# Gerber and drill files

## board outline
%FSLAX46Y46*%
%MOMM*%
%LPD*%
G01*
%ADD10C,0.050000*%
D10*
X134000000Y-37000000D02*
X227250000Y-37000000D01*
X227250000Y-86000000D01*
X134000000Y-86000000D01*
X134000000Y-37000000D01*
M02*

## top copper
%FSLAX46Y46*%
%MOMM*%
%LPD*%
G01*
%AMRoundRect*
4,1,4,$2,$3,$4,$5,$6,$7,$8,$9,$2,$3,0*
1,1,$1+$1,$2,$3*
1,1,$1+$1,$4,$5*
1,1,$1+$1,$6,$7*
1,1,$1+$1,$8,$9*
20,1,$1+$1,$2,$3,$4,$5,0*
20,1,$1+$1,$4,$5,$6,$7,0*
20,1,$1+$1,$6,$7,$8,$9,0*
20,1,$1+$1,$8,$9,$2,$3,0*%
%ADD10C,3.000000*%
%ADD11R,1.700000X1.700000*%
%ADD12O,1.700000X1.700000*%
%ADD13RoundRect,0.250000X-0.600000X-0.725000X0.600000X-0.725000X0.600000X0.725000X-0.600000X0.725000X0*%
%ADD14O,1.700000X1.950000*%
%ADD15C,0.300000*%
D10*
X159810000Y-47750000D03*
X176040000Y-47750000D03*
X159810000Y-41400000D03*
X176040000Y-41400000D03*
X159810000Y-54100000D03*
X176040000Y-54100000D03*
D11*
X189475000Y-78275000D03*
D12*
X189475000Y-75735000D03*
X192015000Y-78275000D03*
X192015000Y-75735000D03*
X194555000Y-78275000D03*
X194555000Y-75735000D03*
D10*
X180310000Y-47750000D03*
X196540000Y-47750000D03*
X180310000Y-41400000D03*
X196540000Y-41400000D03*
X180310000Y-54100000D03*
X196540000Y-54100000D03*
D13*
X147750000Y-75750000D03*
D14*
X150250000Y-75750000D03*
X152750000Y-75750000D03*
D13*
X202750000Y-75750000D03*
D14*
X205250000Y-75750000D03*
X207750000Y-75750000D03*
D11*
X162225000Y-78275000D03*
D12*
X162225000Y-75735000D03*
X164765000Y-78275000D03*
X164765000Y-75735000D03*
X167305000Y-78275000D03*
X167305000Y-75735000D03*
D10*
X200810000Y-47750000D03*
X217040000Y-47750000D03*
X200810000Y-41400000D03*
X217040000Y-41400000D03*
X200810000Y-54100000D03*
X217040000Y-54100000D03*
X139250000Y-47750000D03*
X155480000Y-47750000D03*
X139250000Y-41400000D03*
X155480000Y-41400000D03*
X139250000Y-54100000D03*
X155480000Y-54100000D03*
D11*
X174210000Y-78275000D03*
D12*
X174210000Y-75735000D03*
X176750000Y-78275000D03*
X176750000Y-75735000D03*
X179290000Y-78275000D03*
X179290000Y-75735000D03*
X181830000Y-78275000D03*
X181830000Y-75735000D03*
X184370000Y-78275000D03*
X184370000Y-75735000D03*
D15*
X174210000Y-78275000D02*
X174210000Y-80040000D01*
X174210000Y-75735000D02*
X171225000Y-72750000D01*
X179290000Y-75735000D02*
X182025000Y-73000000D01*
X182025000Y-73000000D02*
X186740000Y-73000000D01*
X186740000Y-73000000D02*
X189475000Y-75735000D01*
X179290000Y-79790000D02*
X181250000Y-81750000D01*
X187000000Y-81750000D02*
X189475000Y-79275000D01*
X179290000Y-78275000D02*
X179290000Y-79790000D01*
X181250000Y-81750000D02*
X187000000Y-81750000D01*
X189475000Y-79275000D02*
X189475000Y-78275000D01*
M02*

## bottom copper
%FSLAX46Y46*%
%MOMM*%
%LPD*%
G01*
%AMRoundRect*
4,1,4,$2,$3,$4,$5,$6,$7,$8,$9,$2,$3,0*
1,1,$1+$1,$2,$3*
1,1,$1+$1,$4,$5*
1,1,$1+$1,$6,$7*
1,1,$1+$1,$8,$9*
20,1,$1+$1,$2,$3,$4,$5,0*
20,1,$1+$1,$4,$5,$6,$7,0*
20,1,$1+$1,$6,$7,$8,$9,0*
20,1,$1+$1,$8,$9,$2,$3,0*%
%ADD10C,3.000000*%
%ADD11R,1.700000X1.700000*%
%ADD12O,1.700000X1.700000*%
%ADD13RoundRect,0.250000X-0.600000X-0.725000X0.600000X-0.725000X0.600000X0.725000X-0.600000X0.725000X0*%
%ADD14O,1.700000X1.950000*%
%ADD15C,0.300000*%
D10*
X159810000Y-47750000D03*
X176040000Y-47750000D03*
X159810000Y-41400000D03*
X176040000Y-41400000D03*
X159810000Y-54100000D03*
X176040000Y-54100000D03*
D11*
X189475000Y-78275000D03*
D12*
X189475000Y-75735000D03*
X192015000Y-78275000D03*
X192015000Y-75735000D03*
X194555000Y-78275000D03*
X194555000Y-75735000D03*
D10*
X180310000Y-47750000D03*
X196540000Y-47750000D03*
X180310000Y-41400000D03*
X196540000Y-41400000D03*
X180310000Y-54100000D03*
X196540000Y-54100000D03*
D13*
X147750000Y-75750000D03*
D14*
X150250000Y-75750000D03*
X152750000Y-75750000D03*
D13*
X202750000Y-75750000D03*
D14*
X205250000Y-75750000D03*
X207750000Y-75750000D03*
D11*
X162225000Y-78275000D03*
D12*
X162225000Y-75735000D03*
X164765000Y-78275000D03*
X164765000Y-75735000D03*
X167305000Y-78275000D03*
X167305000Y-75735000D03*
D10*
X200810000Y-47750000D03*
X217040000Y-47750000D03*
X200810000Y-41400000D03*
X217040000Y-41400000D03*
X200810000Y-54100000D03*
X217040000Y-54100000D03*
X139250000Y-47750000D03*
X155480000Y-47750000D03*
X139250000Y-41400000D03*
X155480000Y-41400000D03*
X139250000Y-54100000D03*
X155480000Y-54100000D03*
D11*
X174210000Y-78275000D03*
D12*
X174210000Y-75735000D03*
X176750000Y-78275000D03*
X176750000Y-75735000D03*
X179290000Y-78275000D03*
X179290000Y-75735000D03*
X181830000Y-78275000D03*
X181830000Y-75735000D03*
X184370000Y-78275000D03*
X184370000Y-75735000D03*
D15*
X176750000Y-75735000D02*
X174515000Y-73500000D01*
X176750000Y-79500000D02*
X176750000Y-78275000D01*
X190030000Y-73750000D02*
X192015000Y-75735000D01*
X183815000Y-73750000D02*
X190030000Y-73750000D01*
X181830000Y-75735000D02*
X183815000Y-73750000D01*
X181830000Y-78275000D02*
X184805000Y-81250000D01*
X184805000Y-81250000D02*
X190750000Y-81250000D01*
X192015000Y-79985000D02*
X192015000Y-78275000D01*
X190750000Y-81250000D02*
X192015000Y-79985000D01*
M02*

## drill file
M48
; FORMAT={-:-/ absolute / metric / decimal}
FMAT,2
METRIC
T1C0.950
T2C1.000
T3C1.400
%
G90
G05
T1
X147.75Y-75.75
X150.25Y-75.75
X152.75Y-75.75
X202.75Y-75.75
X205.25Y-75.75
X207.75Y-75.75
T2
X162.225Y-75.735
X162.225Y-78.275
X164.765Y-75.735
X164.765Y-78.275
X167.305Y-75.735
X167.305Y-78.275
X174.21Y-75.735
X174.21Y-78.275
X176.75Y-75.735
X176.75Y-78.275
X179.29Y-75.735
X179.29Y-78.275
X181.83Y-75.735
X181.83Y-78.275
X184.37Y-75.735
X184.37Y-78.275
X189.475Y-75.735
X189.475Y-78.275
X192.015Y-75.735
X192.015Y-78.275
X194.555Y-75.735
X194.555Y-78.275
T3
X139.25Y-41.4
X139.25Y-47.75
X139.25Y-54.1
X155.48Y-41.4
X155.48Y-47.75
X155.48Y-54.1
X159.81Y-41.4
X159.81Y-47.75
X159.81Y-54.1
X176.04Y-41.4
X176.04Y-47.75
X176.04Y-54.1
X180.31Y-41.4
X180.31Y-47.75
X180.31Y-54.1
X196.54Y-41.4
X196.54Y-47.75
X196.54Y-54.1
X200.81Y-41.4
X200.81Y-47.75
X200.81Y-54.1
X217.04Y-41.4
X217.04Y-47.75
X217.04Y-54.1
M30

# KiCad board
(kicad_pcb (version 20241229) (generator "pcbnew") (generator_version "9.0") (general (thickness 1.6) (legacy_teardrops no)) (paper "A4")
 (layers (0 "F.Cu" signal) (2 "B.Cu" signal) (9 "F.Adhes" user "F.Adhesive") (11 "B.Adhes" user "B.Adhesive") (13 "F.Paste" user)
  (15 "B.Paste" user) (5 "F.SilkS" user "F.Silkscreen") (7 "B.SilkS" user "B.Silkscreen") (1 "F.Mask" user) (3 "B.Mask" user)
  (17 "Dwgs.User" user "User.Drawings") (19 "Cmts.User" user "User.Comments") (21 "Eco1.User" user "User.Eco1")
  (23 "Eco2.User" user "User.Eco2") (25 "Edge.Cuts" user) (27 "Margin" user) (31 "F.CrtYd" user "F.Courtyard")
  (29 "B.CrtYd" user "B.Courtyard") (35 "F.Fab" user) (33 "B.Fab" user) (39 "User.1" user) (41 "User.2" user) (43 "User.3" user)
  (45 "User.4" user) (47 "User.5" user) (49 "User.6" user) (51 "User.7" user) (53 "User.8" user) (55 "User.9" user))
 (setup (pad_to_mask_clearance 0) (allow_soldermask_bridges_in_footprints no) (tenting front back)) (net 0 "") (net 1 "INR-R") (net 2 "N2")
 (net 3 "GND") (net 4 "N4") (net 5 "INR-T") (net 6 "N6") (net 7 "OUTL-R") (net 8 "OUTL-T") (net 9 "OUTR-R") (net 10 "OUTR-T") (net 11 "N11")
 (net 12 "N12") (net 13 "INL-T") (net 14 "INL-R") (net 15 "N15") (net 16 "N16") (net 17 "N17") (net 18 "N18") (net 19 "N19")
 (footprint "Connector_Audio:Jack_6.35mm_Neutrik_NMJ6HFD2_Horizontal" (layer "F.Cu") (at 159.81 54.1 90)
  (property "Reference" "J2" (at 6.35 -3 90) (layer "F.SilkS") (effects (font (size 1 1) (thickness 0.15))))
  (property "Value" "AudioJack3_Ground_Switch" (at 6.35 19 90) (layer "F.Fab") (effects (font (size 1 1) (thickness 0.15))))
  (pad "R" thru_hole circle (at 6.35 0 90) (size 3 3) (drill 1.4) (layers "*.Cu" "*.Mask") (remove_unused_layers no) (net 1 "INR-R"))
  (pad "RN" thru_hole circle (at 6.35 16.23 90) (size 3 3) (drill 1.4) (layers "*.Cu" "*.Mask") (remove_unused_layers no) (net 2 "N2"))
  (pad "S" thru_hole circle (at 12.7 0 90) (size 3 3) (drill 1.4) (layers "*.Cu" "*.Mask") (remove_unused_layers no) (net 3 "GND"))
  (pad "SN" thru_hole circle (at 12.7 16.23 90) (size 3 3) (drill 1.4) (layers "*.Cu" "*.Mask") (remove_unused_layers no) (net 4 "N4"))
  (pad "T" thru_hole circle (at 0 0 90) (size 3 3) (drill 1.4) (layers "*.Cu" "*.Mask") (remove_unused_layers no) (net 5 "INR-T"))
  (pad "TN" thru_hole circle (at 0 16.23 90) (size 3 3) (drill 1.4) (layers "*.Cu" "*.Mask") (remove_unused_layers no) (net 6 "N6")))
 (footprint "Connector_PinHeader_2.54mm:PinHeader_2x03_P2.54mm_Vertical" (layer "F.Cu") (at 189.475 78.275 90)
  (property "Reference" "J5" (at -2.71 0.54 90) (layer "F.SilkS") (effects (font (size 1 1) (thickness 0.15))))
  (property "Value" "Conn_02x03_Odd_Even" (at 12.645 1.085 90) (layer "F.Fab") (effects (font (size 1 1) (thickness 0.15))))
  (pad "1" thru_hole rect (at 0 0 90) (size 1.7 1.7) (drill 1) (layers "*.Cu" "*.Mask") (remove_unused_layers no) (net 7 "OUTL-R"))
  (pad "2" thru_hole oval (at 2.54 0 90) (size 1.7 1.7) (drill 1) (layers "*.Cu" "*.Mask") (remove_unused_layers no) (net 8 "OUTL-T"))
  (pad "3" thru_hole oval (at 0 2.54 90) (size 1.7 1.7) (drill 1) (layers "*.Cu" "*.Mask") (remove_unused_layers no) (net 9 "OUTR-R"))
  (pad "4" thru_hole oval (at 2.54 2.54 90) (size 1.7 1.7) (drill 1) (layers "*.Cu" "*.Mask") (remove_unused_layers no) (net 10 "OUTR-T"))
  (pad "5" thru_hole oval (at 0 5.08 90) (size 1.7 1.7) (drill 1) (layers "*.Cu" "*.Mask") (remove_unused_layers no) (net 3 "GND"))
  (pad "6" thru_hole oval (at 2.54 5.08 90) (size 1.7 1.7) (drill 1) (layers "*.Cu" "*.Mask") (remove_unused_layers no) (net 3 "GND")))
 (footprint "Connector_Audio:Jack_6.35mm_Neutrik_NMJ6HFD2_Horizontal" (layer "F.Cu") (at 180.31 54.1 90)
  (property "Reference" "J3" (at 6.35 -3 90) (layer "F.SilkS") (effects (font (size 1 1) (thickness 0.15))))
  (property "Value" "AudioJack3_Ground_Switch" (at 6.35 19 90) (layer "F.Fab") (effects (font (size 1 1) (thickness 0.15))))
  (pad "R" thru_hole circle (at 6.35 0 90) (size 3 3) (drill 1.4) (layers "*.Cu" "*.Mask") (remove_unused_layers no) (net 9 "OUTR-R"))
  (pad "RN" thru_hole circle (at 6.35 16.23 90) (size 3 3) (drill 1.4) (layers "*.Cu" "*.Mask") (remove_unused_layers no) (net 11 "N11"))
  (pad "S" thru_hole circle (at 12.7 0 90) (size 3 3) (drill 1.4) (layers "*.Cu" "*.Mask") (remove_unused_layers no) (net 3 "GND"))
  (pad "SN" thru_hole circle (at 12.7 16.23 90) (size 3 3) (drill 1.4) (layers "*.Cu" "*.Mask") (remove_unused_layers no) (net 3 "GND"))
  (pad "T" thru_hole circle (at 0 0 90) (size 3 3) (drill 1.4) (layers "*.Cu" "*.Mask") (remove_unused_layers no) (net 10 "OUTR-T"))
  (pad "TN" thru_hole circle (at 0 16.23 90) (size 3 3) (drill 1.4) (layers "*.Cu" "*.Mask") (remove_unused_layers no) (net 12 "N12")))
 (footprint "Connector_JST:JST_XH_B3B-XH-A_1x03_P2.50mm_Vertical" (layer "F.Cu") (at 147.75 75.75)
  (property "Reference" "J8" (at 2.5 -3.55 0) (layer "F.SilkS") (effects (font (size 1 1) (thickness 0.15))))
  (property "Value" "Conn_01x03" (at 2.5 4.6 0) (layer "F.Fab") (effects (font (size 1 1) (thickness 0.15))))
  (pad "1" thru_hole roundrect (at 0 0) (size 1.7 1.95) (drill 0.95) (layers "*.Cu" "*.Mask") (remove_unused_layers no)
   (roundrect_rratio 0.147059) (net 5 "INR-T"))
  (pad "2" thru_hole oval (at 2.5 0) (size 1.7 1.95) (drill 0.95) (layers "*.Cu" "*.Mask") (remove_unused_layers no) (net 3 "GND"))
  (pad "3" thru_hole oval (at 5 0) (size 1.7 1.95) (drill 0.95) (layers "*.Cu" "*.Mask") (remove_unused_layers no) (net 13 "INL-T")))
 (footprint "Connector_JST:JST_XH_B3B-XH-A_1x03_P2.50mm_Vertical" (layer "F.Cu") (at 202.75 75.75)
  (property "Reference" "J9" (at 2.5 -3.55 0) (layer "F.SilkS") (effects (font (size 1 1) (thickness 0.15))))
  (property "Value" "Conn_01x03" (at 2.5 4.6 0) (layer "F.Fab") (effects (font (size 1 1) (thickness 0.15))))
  (pad "1" thru_hole roundrect (at 0 0) (size 1.7 1.95) (drill 0.95) (layers "*.Cu" "*.Mask") (remove_unused_layers no)
   (roundrect_rratio 0.147059) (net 10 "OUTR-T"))
  (pad "2" thru_hole oval (at 2.5 0) (size 1.7 1.95) (drill 0.95) (layers "*.Cu" "*.Mask") (remove_unused_layers no) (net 3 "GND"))
  (pad "3" thru_hole oval (at 5 0) (size 1.7 1.95) (drill 0.95) (layers "*.Cu" "*.Mask") (remove_unused_layers no) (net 8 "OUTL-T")))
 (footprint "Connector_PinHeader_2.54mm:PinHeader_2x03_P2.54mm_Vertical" (layer "F.Cu") (at 162.225 78.275 90)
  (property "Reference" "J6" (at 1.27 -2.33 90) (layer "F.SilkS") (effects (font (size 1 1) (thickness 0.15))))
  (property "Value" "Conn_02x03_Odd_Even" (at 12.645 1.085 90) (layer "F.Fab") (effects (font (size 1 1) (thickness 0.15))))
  (pad "1" thru_hole rect (at 0 0 90) (size 1.7 1.7) (drill 1) (layers "*.Cu" "*.Mask") (remove_unused_layers no) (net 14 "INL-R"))
  (pad "2" thru_hole oval (at 2.54 0 90) (size 1.7 1.7) (drill 1) (layers "*.Cu" "*.Mask") (remove_unused_layers no) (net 13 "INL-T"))
  (pad "3" thru_hole oval (at 0 2.54 90) (size 1.7 1.7) (drill 1) (layers "*.Cu" "*.Mask") (remove_unused_layers no) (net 1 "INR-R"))
  (pad "4" thru_hole oval (at 2.54 2.54 90) (size 1.7 1.7) (drill 1) (layers "*.Cu" "*.Mask") (remove_unused_layers no) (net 5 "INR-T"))
  (pad "5" thru_hole oval (at 0 5.08 90) (size 1.7 1.7) (drill 1) (layers "*.Cu" "*.Mask") (remove_unused_layers no) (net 3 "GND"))
  (pad "6" thru_hole oval (at 2.54 5.08 90) (size 1.7 1.7) (drill 1) (layers "*.Cu" "*.Mask") (remove_unused_layers no) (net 3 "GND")))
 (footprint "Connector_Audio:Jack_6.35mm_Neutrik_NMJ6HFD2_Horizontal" (layer "F.Cu") (at 200.81 54.1 90)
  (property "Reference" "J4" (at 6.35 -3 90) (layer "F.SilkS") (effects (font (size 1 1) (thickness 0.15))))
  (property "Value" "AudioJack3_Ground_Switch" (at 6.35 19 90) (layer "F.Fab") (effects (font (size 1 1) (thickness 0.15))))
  (pad "R" thru_hole circle (at 6.35 0 90) (size 3 3) (drill 1.4) (layers "*.Cu" "*.Mask") (remove_unused_layers no) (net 7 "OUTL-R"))
  (pad "RN" thru_hole circle (at 6.35 16.23 90) (size 3 3) (drill 1.4) (layers "*.Cu" "*.Mask") (remove_unused_layers no) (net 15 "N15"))
  (pad "S" thru_hole circle (at 12.7 0 90) (size 3 3) (drill 1.4) (layers "*.Cu" "*.Mask") (remove_unused_layers no) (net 3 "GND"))
  (pad "SN" thru_hole circle (at 12.7 16.23 90) (size 3 3) (drill 1.4) (layers "*.Cu" "*.Mask") (remove_unused_layers no) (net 3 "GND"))
  (pad "T" thru_hole circle (at 0 0 90) (size 3 3) (drill 1.4) (layers "*.Cu" "*.Mask") (remove_unused_layers no) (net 8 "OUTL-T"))
  (pad "TN" thru_hole circle (at 0 16.23 90) (size 3 3) (drill 1.4) (layers "*.Cu" "*.Mask") (remove_unused_layers no) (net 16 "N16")))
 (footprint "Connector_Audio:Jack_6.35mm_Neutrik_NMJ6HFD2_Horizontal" (layer "F.Cu") (at 139.25 54.1 90)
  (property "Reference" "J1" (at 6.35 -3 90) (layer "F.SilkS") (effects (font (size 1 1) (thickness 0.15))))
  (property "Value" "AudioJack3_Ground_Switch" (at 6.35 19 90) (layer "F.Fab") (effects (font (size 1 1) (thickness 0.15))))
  (pad "R" thru_hole circle (at 6.35 0 90) (size 3 3) (drill 1.4) (layers "*.Cu" "*.Mask") (remove_unused_layers no) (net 14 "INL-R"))
  (pad "RN" thru_hole circle (at 6.35 16.23 90) (size 3 3) (drill 1.4) (layers "*.Cu" "*.Mask") (remove_unused_layers no) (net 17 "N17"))
  (pad "S" thru_hole circle (at 12.7 0 90) (size 3 3) (drill 1.4) (layers "*.Cu" "*.Mask") (remove_unused_layers no) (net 3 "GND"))
  (pad "SN" thru_hole circle (at 12.7 16.23 90) (size 3 3) (drill 1.4) (layers "*.Cu" "*.Mask") (remove_unused_layers no) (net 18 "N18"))
  (pad "T" thru_hole circle (at 0 0 90) (size 3 3) (drill 1.4) (layers "*.Cu" "*.Mask") (remove_unused_layers no) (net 13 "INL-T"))
  (pad "TN" thru_hole circle (at 0 16.23 90) (size 3 3) (drill 1.4) (layers "*.Cu" "*.Mask") (remove_unused_layers no) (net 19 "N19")))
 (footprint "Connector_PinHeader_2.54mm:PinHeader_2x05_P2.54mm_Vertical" (layer "F.Cu") (at 174.21 78.275 90)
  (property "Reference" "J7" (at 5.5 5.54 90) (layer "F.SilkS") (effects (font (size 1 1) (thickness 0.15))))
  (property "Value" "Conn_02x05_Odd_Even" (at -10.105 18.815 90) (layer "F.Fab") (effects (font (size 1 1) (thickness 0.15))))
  (pad "1" thru_hole rect (at 0 0 90) (size 1.7 1.7) (drill 1) (layers "*.Cu" "*.Mask") (remove_unused_layers no) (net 14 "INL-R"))
  (pad "2" thru_hole oval (at 2.54 0 90) (size 1.7 1.7) (drill 1) (layers "*.Cu" "*.Mask") (remove_unused_layers no) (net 13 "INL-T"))
  (pad "3" thru_hole oval (at 0 2.54 90) (size 1.7 1.7) (drill 1) (layers "*.Cu" "*.Mask") (remove_unused_layers no) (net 1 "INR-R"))
  (pad "4" thru_hole oval (at 2.54 2.54 90) (size 1.7 1.7) (drill 1) (layers "*.Cu" "*.Mask") (remove_unused_layers no) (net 5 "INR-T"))
  (pad "5" thru_hole oval (at 0 5.08 90) (size 1.7 1.7) (drill 1) (layers "*.Cu" "*.Mask") (remove_unused_layers no) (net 7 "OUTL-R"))
  (pad "6" thru_hole oval (at 2.54 5.08 90) (size 1.7 1.7) (drill 1) (layers "*.Cu" "*.Mask") (remove_unused_layers no) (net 8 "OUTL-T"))
  (pad "7" thru_hole oval (at 0 7.62 90) (size 1.7 1.7) (drill 1) (layers "*.Cu" "*.Mask") (remove_unused_layers no) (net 9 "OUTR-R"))
  (pad "8" thru_hole oval (at 2.54 7.62 90) (size 1.7 1.7) (drill 1) (layers "*.Cu" "*.Mask") (remove_unused_layers no) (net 10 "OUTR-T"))
  (pad "9" thru_hole oval (at 0 10.16 90) (size 1.7 1.7) (drill 1) (layers "*.Cu" "*.Mask") (remove_unused_layers no) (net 3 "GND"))
  (pad "10" thru_hole oval (at 2.54 10.16 90) (size 1.7 1.7) (drill 1) (layers "*.Cu" "*.Mask") (remove_unused_layers no) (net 3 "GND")))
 (gr_rect (start 134 37) (end 227.25 86) (stroke (width 0.05) (type default)) (fill no) (layer "Edge.Cuts"))
 (segment (start 174.21 78.275) (end 174.21 80.04) (width 0.3) (layer "F.Cu") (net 14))
 (segment (start 174.21 75.735) (end 171.225 72.75) (width 0.3) (layer "F.Cu") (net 13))
 (segment (start 176.75 75.735) (end 174.515 73.5) (width 0.3) (layer "B.Cu") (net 5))
 (segment (start 176.75 79.5) (end 176.75 78.275) (width 0.3) (layer "B.Cu") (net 1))
 (segment (start 190.03 73.75) (end 192.015 75.735) (width 0.3) (layer "B.Cu") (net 10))
 (segment (start 183.815 73.75) (end 190.03 73.75) (width 0.3) (layer "B.Cu") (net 10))
 (segment (start 181.83 75.735) (end 183.815 73.75) (width 0.3) (layer "B.Cu") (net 10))
 (segment (start 181.83 78.275) (end 184.805 81.25) (width 0.3) (layer "B.Cu") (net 9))
 (segment (start 184.805 81.25) (end 190.75 81.25) (width 0.3) (layer "B.Cu") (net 9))
 (segment (start 192.015 79.985) (end 192.015 78.275) (width 0.3) (layer "B.Cu") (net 9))
 (segment (start 190.75 81.25) (end 192.015 79.985) (width 0.3) (layer "B.Cu") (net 9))
 (segment (start 179.29 75.735) (end 182.025 73) (width 0.3) (layer "F.Cu") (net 8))
 (segment (start 182.025 73) (end 186.74 73) (width 0.3) (layer "F.Cu") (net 8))
 (segment (start 186.74 73) (end 189.475 75.735) (width 0.3) (layer "F.Cu") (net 8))
 (segment (start 179.29 79.79) (end 181.25 81.75) (width 0.3) (layer "F.Cu") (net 7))
 (segment (start 187 81.75) (end 189.475 79.275) (width 0.3) (layer "F.Cu") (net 7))
 (segment (start 179.29 78.275) (end 179.29 79.79) (width 0.3) (layer "F.Cu") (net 7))
 (segment (start 181.25 81.75) (end 187 81.75) (width 0.3) (layer "F.Cu") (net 7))
 (segment (start 189.475 79.275) (end 189.475 78.275) (width 0.3) (layer "F.Cu") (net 7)))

